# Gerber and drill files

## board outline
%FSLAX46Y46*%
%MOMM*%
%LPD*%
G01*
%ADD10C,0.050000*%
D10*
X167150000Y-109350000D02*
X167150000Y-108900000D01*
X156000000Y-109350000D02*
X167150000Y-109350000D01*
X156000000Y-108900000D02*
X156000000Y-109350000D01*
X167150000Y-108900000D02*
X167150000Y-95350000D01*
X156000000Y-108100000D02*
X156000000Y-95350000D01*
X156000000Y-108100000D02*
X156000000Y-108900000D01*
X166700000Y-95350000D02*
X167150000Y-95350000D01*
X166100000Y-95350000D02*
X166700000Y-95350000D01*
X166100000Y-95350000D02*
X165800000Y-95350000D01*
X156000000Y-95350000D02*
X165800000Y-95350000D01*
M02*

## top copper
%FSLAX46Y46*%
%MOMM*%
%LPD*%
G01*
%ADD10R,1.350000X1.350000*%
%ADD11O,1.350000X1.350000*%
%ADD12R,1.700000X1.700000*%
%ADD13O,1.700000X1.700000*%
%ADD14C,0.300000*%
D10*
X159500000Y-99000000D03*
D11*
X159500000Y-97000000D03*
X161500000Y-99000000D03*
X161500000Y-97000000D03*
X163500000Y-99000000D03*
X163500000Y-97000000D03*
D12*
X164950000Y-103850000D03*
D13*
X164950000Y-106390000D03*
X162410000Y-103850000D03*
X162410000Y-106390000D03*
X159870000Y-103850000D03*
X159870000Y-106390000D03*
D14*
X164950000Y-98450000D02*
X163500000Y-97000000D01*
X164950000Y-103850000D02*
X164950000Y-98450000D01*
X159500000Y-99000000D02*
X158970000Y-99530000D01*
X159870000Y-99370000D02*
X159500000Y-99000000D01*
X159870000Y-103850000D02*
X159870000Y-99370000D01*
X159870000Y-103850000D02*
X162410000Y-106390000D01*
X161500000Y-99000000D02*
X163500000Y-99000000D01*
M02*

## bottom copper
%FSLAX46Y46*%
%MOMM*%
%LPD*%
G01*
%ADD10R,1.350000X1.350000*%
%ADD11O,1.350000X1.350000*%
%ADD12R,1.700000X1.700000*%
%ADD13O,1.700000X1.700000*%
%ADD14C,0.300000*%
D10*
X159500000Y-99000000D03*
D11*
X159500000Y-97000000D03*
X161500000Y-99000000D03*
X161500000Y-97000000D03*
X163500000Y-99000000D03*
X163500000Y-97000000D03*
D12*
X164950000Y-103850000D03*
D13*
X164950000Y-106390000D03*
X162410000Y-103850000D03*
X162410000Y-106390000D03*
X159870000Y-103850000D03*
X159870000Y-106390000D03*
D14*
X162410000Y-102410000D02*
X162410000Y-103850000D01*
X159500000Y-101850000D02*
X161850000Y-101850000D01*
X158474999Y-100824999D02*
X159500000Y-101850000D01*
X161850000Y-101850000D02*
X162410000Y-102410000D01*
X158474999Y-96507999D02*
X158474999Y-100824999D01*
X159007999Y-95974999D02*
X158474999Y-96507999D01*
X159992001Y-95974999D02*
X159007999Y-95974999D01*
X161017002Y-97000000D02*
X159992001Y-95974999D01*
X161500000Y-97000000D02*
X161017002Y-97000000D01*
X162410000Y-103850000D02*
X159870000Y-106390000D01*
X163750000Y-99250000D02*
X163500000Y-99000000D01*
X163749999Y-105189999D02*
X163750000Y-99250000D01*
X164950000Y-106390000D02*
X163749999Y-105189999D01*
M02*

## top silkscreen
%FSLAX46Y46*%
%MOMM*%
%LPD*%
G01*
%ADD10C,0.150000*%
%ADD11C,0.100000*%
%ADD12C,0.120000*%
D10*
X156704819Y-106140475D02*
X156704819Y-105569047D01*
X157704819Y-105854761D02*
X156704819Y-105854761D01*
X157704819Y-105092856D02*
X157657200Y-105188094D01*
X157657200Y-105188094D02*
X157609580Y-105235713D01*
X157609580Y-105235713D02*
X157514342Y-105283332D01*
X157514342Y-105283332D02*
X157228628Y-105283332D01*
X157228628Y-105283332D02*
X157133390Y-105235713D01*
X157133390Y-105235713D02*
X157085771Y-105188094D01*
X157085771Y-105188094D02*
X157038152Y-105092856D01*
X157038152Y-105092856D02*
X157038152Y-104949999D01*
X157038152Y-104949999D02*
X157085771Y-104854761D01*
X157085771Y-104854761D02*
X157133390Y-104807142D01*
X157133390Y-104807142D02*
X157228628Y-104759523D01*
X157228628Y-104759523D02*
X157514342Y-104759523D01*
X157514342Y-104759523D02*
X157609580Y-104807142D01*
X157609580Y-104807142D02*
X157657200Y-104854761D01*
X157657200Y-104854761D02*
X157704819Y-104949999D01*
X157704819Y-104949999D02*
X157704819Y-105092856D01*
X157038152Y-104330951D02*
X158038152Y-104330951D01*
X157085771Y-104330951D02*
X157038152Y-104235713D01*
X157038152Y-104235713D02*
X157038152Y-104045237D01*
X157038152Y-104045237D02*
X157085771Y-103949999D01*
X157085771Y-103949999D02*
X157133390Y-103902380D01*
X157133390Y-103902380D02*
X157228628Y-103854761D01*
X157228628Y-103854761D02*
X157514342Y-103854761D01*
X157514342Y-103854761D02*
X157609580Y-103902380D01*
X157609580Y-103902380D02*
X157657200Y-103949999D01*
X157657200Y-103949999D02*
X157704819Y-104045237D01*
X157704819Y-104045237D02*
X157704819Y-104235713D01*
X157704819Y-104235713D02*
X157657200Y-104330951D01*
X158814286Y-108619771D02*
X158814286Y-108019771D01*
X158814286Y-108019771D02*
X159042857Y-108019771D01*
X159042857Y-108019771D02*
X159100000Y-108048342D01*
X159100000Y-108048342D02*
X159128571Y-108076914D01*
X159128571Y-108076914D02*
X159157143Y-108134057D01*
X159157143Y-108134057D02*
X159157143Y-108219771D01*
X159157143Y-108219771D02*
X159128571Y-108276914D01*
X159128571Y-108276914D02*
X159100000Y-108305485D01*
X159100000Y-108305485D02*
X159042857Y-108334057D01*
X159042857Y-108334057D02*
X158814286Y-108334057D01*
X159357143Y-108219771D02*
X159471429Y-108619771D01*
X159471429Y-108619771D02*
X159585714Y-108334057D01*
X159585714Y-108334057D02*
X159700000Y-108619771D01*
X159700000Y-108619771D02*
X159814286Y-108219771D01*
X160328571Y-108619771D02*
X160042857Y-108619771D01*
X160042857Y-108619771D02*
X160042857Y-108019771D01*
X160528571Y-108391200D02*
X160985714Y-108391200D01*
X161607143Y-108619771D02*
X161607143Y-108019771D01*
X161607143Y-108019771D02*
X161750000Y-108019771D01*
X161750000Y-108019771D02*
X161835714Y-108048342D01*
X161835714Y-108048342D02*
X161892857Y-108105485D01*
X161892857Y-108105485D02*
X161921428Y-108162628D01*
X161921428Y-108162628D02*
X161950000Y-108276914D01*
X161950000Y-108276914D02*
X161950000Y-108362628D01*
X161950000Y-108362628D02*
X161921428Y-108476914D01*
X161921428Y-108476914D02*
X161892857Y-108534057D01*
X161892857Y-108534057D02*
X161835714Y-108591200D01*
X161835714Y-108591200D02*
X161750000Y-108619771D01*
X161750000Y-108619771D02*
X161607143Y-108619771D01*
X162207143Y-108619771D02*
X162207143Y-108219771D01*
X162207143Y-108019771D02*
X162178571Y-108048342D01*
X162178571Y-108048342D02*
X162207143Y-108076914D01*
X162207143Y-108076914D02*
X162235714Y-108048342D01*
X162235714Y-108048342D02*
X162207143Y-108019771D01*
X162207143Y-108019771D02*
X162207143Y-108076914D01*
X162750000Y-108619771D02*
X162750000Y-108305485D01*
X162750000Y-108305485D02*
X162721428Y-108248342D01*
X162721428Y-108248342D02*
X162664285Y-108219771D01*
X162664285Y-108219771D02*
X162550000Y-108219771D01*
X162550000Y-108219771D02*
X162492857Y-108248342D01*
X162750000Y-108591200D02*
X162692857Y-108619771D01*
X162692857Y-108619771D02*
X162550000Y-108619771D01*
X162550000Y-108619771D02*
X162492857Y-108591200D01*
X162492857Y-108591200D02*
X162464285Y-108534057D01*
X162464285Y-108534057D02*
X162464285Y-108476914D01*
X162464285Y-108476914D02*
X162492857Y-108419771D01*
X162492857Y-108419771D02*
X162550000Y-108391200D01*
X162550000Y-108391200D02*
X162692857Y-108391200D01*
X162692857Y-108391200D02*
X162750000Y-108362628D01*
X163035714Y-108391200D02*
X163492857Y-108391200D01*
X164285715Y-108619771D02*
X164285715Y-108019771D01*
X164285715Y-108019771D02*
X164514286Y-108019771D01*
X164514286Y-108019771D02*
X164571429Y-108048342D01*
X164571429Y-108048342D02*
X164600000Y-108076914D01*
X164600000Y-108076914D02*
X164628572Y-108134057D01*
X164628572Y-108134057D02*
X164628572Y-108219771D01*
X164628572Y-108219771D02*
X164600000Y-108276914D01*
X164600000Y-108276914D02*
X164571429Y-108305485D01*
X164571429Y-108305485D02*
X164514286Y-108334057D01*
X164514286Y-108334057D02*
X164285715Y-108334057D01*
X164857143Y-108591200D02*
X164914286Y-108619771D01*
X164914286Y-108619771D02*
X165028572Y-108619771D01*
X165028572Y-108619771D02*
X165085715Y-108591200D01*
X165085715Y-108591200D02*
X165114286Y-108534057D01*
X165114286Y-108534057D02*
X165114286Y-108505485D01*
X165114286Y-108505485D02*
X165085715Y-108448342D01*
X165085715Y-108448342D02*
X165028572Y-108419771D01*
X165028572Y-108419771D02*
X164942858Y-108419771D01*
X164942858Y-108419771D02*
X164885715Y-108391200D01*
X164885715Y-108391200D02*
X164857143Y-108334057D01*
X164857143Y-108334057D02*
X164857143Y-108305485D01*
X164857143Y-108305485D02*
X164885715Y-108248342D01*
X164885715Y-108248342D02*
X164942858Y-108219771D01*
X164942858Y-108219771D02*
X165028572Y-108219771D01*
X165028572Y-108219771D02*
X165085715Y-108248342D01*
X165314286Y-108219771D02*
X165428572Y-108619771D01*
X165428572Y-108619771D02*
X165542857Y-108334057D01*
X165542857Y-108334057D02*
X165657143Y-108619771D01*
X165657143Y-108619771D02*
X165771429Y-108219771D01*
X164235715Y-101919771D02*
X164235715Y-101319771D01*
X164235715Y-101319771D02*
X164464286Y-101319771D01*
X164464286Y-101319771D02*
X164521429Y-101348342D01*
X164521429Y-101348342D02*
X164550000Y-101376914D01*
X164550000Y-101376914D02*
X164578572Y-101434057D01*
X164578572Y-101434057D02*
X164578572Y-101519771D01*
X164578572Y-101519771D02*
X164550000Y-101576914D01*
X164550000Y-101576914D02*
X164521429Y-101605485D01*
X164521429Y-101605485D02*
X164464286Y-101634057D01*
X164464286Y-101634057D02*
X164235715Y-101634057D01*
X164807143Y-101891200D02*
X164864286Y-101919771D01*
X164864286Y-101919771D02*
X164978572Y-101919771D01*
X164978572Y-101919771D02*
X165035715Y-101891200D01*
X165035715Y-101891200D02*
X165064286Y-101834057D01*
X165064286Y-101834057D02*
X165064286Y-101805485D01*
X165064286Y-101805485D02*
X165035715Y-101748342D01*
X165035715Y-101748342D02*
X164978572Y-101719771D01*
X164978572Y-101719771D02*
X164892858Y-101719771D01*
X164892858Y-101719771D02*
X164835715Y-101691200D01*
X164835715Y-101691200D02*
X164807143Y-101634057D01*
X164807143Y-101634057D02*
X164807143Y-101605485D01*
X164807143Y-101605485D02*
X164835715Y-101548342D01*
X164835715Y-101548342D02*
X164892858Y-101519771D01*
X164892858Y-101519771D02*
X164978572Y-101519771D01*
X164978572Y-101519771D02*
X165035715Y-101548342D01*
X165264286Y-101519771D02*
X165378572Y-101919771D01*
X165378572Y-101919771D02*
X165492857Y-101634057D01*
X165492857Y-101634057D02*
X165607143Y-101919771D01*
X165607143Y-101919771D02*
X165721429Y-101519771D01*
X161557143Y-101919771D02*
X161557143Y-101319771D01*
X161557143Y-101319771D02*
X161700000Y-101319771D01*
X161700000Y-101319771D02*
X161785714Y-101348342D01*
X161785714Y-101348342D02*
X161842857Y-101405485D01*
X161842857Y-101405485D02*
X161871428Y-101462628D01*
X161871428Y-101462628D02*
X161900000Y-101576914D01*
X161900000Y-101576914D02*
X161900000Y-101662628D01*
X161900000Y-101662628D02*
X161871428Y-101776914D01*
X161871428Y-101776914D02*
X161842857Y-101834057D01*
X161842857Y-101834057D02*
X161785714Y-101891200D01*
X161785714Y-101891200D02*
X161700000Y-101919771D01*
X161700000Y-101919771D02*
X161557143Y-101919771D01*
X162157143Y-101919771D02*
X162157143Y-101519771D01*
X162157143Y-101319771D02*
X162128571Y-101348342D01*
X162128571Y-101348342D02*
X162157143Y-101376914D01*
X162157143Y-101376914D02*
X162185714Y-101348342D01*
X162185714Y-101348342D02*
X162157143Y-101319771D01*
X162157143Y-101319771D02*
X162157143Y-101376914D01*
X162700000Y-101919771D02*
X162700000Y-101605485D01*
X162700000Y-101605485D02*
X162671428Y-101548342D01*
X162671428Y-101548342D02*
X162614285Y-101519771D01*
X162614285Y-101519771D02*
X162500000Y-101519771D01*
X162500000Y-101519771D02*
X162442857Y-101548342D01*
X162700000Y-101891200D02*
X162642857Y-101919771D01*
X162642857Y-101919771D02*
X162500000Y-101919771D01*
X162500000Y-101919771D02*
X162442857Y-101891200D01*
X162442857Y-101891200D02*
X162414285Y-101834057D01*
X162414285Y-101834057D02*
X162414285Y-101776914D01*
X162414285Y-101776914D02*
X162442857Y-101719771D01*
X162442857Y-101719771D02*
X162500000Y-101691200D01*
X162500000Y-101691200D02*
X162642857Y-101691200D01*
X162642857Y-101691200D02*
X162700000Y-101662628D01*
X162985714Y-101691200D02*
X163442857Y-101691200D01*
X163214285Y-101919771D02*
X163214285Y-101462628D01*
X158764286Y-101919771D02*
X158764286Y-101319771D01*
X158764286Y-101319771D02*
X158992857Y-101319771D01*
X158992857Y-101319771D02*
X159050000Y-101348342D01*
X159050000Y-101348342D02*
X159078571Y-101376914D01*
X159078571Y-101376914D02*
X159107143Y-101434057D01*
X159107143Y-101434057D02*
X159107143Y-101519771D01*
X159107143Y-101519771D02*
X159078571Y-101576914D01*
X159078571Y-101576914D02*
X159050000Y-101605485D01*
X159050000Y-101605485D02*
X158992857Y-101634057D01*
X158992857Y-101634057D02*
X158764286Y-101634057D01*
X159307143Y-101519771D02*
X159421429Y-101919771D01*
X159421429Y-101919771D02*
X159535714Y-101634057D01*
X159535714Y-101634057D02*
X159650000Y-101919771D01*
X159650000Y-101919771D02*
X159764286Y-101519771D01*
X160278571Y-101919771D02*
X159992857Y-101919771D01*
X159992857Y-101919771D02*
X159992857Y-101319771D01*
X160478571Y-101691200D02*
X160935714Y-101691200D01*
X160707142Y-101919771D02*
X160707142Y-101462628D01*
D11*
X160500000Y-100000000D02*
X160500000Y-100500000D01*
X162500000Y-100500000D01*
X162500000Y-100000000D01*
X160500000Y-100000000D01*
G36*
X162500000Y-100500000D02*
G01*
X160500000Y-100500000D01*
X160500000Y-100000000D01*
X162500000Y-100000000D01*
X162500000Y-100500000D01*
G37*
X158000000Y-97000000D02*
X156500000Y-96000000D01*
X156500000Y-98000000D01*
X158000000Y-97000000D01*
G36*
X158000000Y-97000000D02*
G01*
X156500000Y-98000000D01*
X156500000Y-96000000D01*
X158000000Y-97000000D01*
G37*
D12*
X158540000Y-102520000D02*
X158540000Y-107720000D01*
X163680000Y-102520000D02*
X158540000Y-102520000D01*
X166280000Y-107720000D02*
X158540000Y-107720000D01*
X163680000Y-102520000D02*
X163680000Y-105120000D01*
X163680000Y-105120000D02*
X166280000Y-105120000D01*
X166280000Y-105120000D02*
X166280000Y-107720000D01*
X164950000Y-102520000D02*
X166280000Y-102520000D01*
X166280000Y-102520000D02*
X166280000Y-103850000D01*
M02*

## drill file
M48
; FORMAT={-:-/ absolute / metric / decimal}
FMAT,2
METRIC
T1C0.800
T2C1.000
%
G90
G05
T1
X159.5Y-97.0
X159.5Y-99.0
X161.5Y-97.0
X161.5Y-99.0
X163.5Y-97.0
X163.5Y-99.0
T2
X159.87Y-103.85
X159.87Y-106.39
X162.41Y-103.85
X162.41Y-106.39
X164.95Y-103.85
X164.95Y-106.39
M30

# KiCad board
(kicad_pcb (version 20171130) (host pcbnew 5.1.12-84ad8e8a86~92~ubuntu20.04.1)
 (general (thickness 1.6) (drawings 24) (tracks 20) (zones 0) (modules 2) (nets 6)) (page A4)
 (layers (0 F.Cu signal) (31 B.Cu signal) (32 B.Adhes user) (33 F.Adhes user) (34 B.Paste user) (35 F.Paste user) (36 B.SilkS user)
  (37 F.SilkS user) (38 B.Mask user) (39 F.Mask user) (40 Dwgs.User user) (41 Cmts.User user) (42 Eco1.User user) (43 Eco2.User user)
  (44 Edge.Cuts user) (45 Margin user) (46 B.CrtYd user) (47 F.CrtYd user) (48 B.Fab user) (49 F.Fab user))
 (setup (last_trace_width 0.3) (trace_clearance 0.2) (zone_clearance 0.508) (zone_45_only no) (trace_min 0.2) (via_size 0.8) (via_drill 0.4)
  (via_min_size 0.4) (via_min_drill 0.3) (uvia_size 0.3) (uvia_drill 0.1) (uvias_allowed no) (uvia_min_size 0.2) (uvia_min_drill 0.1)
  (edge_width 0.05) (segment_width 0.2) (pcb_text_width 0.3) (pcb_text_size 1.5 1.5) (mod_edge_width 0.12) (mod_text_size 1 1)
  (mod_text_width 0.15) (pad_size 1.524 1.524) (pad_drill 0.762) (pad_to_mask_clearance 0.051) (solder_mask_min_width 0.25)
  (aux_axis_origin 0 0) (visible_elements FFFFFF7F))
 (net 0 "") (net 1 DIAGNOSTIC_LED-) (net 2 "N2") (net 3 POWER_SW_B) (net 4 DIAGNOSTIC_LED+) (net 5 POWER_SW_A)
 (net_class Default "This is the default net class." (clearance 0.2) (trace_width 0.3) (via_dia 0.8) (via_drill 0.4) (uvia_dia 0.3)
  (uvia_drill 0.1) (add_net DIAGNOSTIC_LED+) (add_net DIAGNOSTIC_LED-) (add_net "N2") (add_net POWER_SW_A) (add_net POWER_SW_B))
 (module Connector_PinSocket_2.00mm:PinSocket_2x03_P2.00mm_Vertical (layer B.Cu) (at 159.5 99 270)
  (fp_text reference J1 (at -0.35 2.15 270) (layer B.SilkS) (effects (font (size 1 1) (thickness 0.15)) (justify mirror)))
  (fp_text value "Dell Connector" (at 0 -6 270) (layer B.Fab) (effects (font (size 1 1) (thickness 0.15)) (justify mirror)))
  (pad 1 thru_hole rect (at 0 0 270) (size 1.35 1.35) (drill 0.8) (layers *.Cu *.Mask) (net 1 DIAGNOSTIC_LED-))
  (pad 2 thru_hole oval (at -2 0 270) (size 1.35 1.35) (drill 0.8) (layers *.Cu *.Mask) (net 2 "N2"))
  (pad 3 thru_hole oval (at 0 -2 270) (size 1.35 1.35) (drill 0.8) (layers *.Cu *.Mask) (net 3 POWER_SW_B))
  (pad 4 thru_hole oval (at -2 -2 270) (size 1.35 1.35) (drill 0.8) (layers *.Cu *.Mask) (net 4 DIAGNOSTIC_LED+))
  (pad 5 thru_hole oval (at 0 -4 270) (size 1.35 1.35) (drill 0.8) (layers *.Cu *.Mask) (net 3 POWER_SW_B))
  (pad 6 thru_hole oval (at -2 -4 270) (size 1.35 1.35) (drill 0.8) (layers *.Cu *.Mask) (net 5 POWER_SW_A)))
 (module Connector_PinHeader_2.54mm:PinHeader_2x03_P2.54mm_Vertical (layer F.Cu) (at 164.95 103.85 270)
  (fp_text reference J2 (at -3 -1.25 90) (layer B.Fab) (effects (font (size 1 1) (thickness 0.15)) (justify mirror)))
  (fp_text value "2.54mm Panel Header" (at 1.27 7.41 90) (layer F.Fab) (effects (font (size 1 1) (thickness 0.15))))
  (fp_line (start -1.33 6.41) (end 3.87 6.41) (layer F.SilkS) (width 0.12))
  (fp_line (start -1.33 1.27) (end -1.33 6.41) (layer F.SilkS) (width 0.12))
  (fp_line (start 3.87 -1.33) (end 3.87 6.41) (layer F.SilkS) (width 0.12))
  (fp_line (start -1.33 1.27) (end 1.27 1.27) (layer F.SilkS) (width 0.12))
  (fp_line (start 1.27 1.27) (end 1.27 -1.33) (layer F.SilkS) (width 0.12))
  (fp_line (start 1.27 -1.33) (end 3.87 -1.33) (layer F.SilkS) (width 0.12))
  (fp_line (start -1.33 0) (end -1.33 -1.33) (layer F.SilkS) (width 0.12))
  (fp_line (start -1.33 -1.33) (end 0 -1.33) (layer F.SilkS) (width 0.12))
  (pad 1 thru_hole rect (at 0 0 270) (size 1.7 1.7) (drill 1) (layers *.Cu *.Mask) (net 5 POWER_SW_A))
  (pad 2 thru_hole oval (at 2.54 0 270) (size 1.7 1.7) (drill 1) (layers *.Cu *.Mask) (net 3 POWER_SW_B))
  (pad 3 thru_hole oval (at 0 2.54 270) (size 1.7 1.7) (drill 1) (layers *.Cu *.Mask) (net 4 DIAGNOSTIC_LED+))
  (pad 4 thru_hole oval (at 2.54 2.54 270) (size 1.7 1.7) (drill 1) (layers *.Cu *.Mask) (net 1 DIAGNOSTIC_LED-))
  (pad 5 thru_hole oval (at 0 5.08 270) (size 1.7 1.7) (drill 1) (layers *.Cu *.Mask) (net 1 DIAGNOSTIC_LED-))
  (pad 6 thru_hole oval (at 2.54 5.08 270) (size 1.7 1.7) (drill 1) (layers *.Cu *.Mask) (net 4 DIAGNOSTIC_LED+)))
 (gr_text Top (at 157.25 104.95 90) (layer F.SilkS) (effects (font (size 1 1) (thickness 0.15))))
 (gr_line (start 167.15 109.35) (end 167.15 108.9) (layer Edge.Cuts) (width 0.05))
 (gr_line (start 156 109.35) (end 167.15 109.35) (layer Edge.Cuts) (width 0.05))
 (gr_line (start 156 108.9) (end 156 109.35) (layer Edge.Cuts) (width 0.05))
 (gr_line (start 167.15 108.9) (end 167.15 95.35) (layer Edge.Cuts) (width 0.05))
 (gr_line (start 156 108.1) (end 156 95.35) (layer Edge.Cuts) (width 0.05))
 (gr_line (start 156 108.1) (end 156 108.9) (layer Edge.Cuts) (width 0.05))
 (gr_line (start 166.7 95.35) (end 167.15 95.35) (layer Edge.Cuts) (width 0.05))
 (gr_line (start 166.1 95.35) (end 166.7 95.35) (layer Edge.Cuts) (width 0.05))
 (gr_line (start 166.1 95.35) (end 165.8 95.35) (layer Edge.Cuts) (width 0.05))
 (gr_line (start 156 95.35) (end 165.8 95.35) (layer Edge.Cuts) (width 0.05))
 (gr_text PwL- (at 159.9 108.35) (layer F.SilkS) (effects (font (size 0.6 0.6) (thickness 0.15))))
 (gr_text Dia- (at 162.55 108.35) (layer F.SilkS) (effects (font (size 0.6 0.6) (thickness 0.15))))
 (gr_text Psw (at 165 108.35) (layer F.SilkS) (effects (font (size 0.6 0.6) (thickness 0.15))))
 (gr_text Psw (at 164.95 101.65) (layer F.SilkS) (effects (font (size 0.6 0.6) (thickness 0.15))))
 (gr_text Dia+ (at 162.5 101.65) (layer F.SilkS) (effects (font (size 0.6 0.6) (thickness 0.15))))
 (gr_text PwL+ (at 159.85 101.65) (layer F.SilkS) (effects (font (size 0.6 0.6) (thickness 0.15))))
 (gr_poly (pts (xy 160.5 100) (xy 160.5 100.5) (xy 162.5 100.5) (xy 162.5 100)) (layer F.SilkS) (width 0.1))
 (gr_poly (pts (xy 158 97) (xy 156.5 96) (xy 156.5 98)) (layer F.SilkS) (width 0.1))
 (segment (start 164.95 98.45) (end 163.5 97) (width 0.3) (layer F.Cu) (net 5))
 (segment (start 164.95 103.85) (end 164.95 98.45) (width 0.3) (layer F.Cu) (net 5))
 (segment (start 162.41 102.41) (end 162.41 103.85) (width 0.3) (layer B.Cu) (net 4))
 (segment (start 159.5 101.85) (end 161.85 101.85) (width 0.3) (layer B.Cu) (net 4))
 (segment (start 158.474999 100.824999) (end 159.5 101.85) (width 0.3) (layer B.Cu) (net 4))
 (segment (start 161.85 101.85) (end 162.41 102.41) (width 0.3) (layer B.Cu) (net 4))
 (segment (start 158.474999 96.507999) (end 158.474999 100.824999) (width 0.3) (layer B.Cu) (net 4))
 (segment (start 159.007999 95.974999) (end 158.474999 96.507999) (width 0.3) (layer B.Cu) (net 4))
 (segment (start 159.992001 95.974999) (end 159.007999 95.974999) (width 0.3) (layer B.Cu) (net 4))
 (segment (start 161.017002 97) (end 159.992001 95.974999) (width 0.3) (layer B.Cu) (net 4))
 (segment (start 161.5 97) (end 161.017002 97) (width 0.3) (layer B.Cu) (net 4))
 (segment (start 162.41 103.85) (end 159.87 106.39) (width 0.3) (layer B.Cu) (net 4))
 (segment (start 159.5 99) (end 158.97 99.53) (width 0.3) (layer F.Cu) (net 1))
 (segment (start 159.87 99.37) (end 159.5 99) (width 0.3) (layer F.Cu) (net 1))
 (segment (start 159.87 103.85) (end 159.87 99.37) (width 0.3) (layer F.Cu) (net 1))
 (segment (start 159.87 103.85) (end 162.41 106.39) (width 0.3) (layer F.Cu) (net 1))
 (segment (start 161.5 99) (end 163.5 99) (width 0.3) (layer F.Cu) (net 3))
 (segment (start 163.75 99.25) (end 163.5 99) (width 0.3) (layer B.Cu) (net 3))
 (segment (start 163.749999 105.189999) (end 163.75 99.25) (width 0.3) (layer B.Cu) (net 3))
 (segment (start 164.95 106.39) (end 163.749999 105.189999) (width 0.3) (layer B.Cu) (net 3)))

